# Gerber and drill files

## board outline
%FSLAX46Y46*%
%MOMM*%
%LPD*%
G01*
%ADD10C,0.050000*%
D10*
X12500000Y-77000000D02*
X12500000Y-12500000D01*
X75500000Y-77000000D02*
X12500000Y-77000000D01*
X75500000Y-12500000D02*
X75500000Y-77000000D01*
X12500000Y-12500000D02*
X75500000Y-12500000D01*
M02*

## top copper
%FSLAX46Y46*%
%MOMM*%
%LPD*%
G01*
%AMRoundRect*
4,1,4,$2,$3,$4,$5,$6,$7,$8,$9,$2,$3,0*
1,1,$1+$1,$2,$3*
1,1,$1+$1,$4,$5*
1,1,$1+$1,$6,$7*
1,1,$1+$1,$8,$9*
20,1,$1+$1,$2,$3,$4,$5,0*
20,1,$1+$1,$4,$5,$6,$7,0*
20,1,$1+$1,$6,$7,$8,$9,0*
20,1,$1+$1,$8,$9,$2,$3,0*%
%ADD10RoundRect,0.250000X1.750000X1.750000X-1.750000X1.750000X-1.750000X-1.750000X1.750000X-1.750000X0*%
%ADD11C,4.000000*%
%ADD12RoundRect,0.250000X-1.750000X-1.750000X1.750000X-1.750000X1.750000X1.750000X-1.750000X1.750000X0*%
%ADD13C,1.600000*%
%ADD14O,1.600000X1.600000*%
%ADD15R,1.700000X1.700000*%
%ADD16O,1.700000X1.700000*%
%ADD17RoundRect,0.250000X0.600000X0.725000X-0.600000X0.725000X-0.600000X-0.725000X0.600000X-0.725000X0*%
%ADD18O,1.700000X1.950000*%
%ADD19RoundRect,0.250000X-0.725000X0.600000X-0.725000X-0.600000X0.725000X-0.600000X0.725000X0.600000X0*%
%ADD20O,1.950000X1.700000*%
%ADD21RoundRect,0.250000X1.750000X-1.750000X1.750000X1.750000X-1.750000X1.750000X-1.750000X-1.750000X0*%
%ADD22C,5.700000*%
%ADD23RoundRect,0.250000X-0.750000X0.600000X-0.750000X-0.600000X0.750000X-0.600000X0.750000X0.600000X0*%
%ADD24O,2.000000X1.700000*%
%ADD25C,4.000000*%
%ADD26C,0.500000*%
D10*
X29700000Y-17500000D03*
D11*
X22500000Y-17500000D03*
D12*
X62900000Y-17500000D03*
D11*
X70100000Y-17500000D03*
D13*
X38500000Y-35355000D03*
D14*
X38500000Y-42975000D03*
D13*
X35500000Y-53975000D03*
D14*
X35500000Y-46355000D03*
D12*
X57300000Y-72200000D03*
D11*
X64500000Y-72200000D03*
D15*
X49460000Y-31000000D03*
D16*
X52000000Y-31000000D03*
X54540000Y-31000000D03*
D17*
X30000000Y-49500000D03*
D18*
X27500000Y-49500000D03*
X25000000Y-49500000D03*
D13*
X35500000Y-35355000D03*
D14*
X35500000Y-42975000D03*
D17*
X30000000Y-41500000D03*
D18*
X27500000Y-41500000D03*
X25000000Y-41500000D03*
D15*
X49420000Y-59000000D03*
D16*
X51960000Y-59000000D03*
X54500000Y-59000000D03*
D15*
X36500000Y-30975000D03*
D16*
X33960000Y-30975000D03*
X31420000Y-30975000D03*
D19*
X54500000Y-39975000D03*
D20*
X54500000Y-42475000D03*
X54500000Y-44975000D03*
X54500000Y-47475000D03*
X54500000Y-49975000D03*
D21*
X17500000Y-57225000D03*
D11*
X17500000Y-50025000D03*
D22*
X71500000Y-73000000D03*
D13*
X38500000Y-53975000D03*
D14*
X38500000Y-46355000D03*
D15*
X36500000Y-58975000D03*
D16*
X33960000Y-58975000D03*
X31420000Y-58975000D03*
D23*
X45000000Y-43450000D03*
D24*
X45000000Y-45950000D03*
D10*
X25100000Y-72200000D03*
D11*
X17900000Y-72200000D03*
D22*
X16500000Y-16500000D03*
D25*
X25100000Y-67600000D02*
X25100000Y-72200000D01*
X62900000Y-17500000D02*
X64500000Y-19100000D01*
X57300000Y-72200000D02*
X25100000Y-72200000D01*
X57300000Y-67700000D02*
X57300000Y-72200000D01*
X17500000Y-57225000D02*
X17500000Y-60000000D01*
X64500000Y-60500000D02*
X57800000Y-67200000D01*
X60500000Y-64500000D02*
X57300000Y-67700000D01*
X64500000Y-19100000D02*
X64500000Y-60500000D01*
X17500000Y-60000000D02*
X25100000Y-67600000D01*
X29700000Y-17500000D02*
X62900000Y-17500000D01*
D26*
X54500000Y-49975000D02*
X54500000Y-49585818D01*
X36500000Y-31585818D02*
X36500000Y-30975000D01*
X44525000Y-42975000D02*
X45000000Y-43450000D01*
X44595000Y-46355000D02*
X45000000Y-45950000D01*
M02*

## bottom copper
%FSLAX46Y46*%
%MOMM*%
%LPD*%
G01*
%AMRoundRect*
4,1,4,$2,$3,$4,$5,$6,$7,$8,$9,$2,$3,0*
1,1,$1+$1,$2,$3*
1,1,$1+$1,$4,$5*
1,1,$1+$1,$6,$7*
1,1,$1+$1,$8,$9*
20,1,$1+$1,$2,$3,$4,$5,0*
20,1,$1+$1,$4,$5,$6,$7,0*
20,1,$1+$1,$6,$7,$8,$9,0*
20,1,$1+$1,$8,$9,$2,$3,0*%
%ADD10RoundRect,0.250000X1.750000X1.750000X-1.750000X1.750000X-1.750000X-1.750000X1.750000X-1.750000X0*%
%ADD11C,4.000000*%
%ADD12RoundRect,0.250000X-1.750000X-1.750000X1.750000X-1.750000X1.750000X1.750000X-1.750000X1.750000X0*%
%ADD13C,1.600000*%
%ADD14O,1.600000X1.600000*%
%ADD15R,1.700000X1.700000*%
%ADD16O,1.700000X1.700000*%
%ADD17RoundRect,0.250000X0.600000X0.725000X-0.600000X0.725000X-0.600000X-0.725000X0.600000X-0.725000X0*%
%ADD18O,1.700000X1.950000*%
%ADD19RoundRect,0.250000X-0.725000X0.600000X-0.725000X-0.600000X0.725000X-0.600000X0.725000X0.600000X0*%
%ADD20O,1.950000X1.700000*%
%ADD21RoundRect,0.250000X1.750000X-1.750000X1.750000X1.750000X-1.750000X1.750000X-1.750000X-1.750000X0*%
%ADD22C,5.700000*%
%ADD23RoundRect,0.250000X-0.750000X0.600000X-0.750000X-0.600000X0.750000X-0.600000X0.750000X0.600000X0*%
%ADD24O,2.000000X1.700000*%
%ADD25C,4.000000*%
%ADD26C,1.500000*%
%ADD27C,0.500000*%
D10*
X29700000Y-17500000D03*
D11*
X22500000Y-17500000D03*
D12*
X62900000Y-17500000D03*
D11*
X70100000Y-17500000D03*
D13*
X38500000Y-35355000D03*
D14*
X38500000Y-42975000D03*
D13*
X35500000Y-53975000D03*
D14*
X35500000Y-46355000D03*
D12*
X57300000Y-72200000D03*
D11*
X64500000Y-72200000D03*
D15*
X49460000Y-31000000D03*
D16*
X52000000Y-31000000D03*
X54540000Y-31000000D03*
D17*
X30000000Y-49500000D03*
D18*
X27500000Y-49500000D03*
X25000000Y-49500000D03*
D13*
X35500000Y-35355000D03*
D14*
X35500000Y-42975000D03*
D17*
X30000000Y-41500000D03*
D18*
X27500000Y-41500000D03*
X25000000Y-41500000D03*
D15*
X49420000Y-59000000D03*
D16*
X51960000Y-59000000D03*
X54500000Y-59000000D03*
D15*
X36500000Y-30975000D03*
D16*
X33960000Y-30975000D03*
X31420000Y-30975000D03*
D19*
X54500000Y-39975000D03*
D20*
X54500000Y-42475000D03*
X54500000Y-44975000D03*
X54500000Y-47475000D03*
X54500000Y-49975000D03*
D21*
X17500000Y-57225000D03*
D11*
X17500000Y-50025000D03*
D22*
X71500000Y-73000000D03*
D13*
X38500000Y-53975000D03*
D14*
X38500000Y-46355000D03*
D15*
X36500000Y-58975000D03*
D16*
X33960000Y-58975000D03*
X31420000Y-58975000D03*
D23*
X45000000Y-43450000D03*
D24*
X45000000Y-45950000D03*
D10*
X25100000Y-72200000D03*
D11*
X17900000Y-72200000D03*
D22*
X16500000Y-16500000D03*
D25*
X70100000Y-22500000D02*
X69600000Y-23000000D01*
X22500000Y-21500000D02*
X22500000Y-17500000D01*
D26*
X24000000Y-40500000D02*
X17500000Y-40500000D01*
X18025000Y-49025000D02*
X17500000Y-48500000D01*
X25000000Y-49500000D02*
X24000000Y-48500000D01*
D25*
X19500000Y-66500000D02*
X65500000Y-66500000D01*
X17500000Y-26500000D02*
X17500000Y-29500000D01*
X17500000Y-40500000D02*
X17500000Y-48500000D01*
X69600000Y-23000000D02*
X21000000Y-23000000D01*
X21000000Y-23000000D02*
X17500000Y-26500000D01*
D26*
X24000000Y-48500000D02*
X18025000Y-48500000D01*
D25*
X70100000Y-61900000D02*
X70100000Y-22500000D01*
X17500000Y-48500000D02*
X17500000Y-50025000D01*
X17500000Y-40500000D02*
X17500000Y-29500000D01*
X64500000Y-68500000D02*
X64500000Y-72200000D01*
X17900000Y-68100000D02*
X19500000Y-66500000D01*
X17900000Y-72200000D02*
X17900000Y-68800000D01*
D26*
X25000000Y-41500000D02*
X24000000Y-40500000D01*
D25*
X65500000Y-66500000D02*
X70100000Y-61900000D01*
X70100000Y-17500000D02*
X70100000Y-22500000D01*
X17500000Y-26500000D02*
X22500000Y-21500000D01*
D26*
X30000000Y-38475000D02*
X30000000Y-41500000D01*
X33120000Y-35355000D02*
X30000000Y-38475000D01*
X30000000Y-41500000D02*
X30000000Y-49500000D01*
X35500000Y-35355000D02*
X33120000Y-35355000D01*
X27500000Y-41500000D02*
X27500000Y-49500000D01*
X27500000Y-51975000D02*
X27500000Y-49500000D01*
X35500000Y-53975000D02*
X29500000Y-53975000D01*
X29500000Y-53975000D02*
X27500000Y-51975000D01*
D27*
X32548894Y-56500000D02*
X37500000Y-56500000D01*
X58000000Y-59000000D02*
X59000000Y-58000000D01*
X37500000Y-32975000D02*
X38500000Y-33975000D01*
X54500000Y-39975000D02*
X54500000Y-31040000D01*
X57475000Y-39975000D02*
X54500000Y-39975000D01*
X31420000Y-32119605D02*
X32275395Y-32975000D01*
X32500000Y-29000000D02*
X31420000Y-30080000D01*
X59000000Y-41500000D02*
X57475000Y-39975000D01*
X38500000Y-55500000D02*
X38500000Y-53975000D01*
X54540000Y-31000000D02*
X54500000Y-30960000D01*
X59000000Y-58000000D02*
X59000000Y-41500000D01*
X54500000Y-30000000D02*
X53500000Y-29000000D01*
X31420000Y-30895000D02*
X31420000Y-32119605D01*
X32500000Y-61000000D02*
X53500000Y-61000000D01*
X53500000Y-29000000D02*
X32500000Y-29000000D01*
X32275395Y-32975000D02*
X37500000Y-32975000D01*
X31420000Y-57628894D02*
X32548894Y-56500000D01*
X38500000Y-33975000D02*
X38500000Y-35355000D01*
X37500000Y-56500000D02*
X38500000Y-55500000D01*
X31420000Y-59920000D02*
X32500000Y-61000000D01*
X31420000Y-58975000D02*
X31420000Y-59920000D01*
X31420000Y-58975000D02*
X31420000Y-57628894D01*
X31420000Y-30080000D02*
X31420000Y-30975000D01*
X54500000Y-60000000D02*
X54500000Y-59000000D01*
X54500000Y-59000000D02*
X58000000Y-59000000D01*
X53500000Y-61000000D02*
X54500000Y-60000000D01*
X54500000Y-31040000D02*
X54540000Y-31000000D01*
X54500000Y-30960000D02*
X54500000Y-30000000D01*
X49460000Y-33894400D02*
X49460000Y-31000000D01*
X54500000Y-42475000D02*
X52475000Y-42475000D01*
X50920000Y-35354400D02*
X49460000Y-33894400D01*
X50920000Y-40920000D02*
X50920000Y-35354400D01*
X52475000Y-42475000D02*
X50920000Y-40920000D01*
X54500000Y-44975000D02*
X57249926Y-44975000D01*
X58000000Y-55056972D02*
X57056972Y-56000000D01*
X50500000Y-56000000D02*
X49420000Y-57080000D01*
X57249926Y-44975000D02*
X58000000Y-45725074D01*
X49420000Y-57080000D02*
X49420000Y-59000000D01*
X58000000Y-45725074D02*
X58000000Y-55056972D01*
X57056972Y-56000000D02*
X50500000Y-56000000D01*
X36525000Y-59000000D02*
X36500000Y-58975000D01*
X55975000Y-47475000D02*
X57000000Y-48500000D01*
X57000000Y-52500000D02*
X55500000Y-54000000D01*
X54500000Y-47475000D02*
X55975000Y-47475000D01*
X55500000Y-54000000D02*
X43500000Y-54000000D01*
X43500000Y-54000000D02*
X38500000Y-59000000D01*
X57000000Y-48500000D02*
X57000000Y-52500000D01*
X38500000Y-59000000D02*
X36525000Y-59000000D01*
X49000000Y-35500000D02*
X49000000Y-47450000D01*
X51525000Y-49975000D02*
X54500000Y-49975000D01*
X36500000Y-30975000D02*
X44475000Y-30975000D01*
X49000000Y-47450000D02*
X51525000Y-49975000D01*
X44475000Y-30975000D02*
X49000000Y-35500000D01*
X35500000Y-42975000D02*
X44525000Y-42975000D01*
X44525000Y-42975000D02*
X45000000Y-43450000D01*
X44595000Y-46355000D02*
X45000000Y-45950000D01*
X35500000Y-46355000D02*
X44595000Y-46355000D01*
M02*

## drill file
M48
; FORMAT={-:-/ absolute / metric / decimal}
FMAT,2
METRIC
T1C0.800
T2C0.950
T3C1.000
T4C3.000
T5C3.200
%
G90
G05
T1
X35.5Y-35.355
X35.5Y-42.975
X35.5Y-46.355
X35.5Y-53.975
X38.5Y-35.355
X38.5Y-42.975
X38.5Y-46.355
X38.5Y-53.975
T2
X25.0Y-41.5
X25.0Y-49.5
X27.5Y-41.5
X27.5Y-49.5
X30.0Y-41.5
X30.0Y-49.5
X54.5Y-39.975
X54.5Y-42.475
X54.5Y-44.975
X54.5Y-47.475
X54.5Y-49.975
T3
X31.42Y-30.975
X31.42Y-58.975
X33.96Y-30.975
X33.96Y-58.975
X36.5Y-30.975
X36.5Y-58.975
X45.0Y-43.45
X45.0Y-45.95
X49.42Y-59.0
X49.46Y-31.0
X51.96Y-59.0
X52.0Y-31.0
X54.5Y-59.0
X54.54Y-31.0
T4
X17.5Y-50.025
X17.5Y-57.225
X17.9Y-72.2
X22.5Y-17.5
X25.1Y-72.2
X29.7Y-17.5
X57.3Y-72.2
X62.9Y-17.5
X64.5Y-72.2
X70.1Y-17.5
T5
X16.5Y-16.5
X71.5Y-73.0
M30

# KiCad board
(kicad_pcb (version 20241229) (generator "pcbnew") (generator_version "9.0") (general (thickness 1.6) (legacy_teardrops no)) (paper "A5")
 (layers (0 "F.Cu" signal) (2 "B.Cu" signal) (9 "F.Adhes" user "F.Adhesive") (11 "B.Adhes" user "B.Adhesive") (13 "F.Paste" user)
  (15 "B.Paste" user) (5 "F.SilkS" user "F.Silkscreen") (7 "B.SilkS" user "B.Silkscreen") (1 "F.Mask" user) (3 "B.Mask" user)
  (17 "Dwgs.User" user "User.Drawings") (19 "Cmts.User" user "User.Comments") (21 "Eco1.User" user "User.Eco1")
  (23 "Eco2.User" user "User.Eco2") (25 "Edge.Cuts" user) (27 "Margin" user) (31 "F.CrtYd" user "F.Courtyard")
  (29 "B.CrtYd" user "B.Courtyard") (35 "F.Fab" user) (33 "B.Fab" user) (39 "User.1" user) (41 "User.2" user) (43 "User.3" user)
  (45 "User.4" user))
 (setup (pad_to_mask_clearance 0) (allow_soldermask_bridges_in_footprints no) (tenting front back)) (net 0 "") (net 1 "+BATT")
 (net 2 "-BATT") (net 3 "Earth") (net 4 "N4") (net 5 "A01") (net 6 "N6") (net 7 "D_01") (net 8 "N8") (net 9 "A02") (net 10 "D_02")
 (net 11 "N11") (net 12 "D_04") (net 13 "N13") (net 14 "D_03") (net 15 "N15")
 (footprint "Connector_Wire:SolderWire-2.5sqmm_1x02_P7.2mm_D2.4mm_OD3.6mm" (layer "F.Cu") (at 29.7 17.5 180)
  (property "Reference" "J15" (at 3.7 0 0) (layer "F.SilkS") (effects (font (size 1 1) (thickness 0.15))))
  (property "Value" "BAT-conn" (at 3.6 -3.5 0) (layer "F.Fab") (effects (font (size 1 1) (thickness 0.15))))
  (pad "1" thru_hole roundrect (at 0 0 180) (size 4 4) (drill 3) (layers "*.Cu" "*.Mask") (remove_unused_layers no)
   (roundrect_rratio 0.0625) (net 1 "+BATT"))
  (pad "2" thru_hole circle (at 7.2 0 180) (size 4 4) (drill 3) (layers "*.Cu" "*.Mask") (remove_unused_layers no) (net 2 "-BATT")))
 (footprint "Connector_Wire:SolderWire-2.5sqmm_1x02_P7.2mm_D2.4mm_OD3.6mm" (layer "F.Cu") (at 62.9 17.5)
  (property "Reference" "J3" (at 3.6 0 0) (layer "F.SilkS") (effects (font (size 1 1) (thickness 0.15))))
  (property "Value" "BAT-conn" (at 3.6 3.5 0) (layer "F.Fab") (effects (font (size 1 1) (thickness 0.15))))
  (pad "1" thru_hole roundrect (at 0 0) (size 4 4) (drill 3) (layers "*.Cu" "*.Mask") (remove_unused_layers no) (roundrect_rratio 0.0625)
   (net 1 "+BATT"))
  (pad "2" thru_hole circle (at 7.2 0) (size 4 4) (drill 3) (layers "*.Cu" "*.Mask") (remove_unused_layers no) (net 2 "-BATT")))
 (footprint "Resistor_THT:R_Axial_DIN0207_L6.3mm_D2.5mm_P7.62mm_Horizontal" (layer "F.Cu") (at 38.5 35.355 -90)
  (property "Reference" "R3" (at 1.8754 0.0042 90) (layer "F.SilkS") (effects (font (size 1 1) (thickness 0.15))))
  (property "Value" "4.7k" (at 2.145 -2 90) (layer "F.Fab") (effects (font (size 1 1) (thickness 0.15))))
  (pad "1" thru_hole circle (at 0 0 270) (size 1.6 1.6) (drill 0.8) (layers "*.Cu" "*.Mask") (remove_unused_layers no) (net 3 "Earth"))
  (pad "2" thru_hole oval (at 7.62 0 270) (size 1.6 1.6) (drill 0.8) (layers "*.Cu" "*.Mask") (remove_unused_layers no) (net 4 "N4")))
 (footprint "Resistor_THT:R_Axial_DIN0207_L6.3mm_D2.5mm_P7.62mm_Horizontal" (layer "F.Cu") (at 35.5 53.975 90)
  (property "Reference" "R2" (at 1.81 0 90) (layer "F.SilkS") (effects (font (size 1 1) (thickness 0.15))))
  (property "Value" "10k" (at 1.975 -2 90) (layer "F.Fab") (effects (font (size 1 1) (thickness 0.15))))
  (pad "1" thru_hole circle (at 0 0 90) (size 1.6 1.6) (drill 0.8) (layers "*.Cu" "*.Mask") (remove_unused_layers no) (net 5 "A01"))
  (pad "2" thru_hole oval (at 7.62 0 90) (size 1.6 1.6) (drill 0.8) (layers "*.Cu" "*.Mask") (remove_unused_layers no) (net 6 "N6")))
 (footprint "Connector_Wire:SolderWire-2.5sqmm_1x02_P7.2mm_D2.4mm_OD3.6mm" (layer "F.Cu") (at 57.3 72.2)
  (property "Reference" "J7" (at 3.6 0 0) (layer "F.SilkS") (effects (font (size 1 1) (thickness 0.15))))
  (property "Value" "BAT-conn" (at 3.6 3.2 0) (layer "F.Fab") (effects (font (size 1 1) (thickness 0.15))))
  (pad "1" thru_hole roundrect (at 0 0) (size 4 4) (drill 3) (layers "*.Cu" "*.Mask") (remove_unused_layers no) (roundrect_rratio 0.0625)
   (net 1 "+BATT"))
  (pad "2" thru_hole circle (at 7.2 0) (size 4 4) (drill 3) (layers "*.Cu" "*.Mask") (remove_unused_layers no) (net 2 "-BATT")))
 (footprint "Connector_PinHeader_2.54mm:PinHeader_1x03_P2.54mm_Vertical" (layer "F.Cu") (at 49.46 31 90)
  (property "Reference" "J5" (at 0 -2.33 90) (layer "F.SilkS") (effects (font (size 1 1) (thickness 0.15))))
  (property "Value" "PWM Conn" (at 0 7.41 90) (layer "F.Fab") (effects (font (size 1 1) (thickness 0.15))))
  (pad "1" thru_hole rect (at 0 0 90) (size 1.7 1.7) (drill 1) (layers "*.Cu" "*.Mask") (remove_unused_layers no) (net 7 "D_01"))
  (pad "2" thru_hole oval (at 0 2.54 90) (size 1.7 1.7) (drill 1) (layers "*.Cu" "*.Mask") (remove_unused_layers no) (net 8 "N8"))
  (pad "3" thru_hole oval (at 0 5.08 90) (size 1.7 1.7) (drill 1) (layers "*.Cu" "*.Mask") (remove_unused_layers no) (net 3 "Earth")))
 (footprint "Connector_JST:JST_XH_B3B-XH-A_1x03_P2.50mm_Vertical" (layer "F.Cu") (at 30 49.5 180)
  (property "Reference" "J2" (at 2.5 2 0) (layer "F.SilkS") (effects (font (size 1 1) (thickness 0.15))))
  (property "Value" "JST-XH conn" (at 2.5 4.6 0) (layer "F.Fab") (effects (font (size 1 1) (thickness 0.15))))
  (pad "1" thru_hole roundrect (at 0 0 180) (size 1.7 1.95) (drill 0.95) (layers "*.Cu" "*.Mask") (remove_unused_layers no)
   (roundrect_rratio 0.147059) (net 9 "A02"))
  (pad "2" thru_hole oval (at 2.5 0 180) (size 1.7 1.95) (drill 0.95) (layers "*.Cu" "*.Mask") (remove_unused_layers no) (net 5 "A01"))
  (pad "3" thru_hole oval (at 5 0 180) (size 1.7 1.95) (drill 0.95) (layers "*.Cu" "*.Mask") (remove_unused_layers no) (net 2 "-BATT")))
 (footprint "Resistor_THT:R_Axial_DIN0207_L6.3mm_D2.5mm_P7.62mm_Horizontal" (layer "F.Cu") (at 35.5 35.355 -90)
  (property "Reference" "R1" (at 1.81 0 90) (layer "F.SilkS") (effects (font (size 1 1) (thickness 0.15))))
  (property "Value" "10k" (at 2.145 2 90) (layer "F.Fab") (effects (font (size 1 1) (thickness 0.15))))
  (pad "1" thru_hole circle (at 0 0 270) (size 1.6 1.6) (drill 0.8) (layers "*.Cu" "*.Mask") (remove_unused_layers no) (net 9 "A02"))
  (pad "2" thru_hole oval (at 7.62 0 270) (size 1.6 1.6) (drill 0.8) (layers "*.Cu" "*.Mask") (remove_unused_layers no) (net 4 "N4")))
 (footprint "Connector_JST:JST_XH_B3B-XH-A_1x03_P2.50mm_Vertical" (layer "F.Cu") (at 30 41.5 180)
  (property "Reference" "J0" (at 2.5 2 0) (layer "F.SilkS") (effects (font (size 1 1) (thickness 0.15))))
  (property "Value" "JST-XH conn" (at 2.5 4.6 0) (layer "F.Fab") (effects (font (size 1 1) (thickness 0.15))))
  (pad "1" thru_hole roundrect (at 0 0 180) (size 1.7 1.95) (drill 0.95) (layers "*.Cu" "*.Mask") (remove_unused_layers no)
   (roundrect_rratio 0.147059) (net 9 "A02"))
  (pad "2" thru_hole oval (at 2.5 0 180) (size 1.7 1.95) (drill 0.95) (layers "*.Cu" "*.Mask") (remove_unused_layers no) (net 5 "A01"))
  (pad "3" thru_hole oval (at 5 0 180) (size 1.7 1.95) (drill 0.95) (layers "*.Cu" "*.Mask") (remove_unused_layers no) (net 2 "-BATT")))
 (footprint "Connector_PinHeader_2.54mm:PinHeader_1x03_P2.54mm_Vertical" (layer "F.Cu") (at 49.42 59 90)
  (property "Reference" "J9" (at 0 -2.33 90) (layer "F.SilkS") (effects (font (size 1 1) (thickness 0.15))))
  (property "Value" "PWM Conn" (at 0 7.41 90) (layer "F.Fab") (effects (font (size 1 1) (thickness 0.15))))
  (pad "1" thru_hole rect (at 0 0 90) (size 1.7 1.7) (drill 1) (layers "*.Cu" "*.Mask") (remove_unused_layers no) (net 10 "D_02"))
  (pad "2" thru_hole oval (at 0 2.54 90) (size 1.7 1.7) (drill 1) (layers "*.Cu" "*.Mask") (remove_unused_layers no) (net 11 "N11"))
  (pad "3" thru_hole oval (at 0 5.08 90) (size 1.7 1.7) (drill 1) (layers "*.Cu" "*.Mask") (remove_unused_layers no) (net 3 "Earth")))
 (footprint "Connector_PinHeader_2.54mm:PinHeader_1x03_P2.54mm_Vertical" (layer "F.Cu") (at 36.5 30.975 -90)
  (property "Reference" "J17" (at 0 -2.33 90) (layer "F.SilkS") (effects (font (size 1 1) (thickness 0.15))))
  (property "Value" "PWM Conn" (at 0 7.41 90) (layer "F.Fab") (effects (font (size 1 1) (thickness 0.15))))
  (pad "1" thru_hole rect (at 0 0 270) (size 1.7 1.7) (drill 1) (layers "*.Cu" "*.Mask") (remove_unused_layers no) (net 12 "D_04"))
  (pad "2" thru_hole oval (at 0 2.54 270) (size 1.7 1.7) (drill 1) (layers "*.Cu" "*.Mask") (remove_unused_layers no) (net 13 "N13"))
  (pad "3" thru_hole oval (at 0 5.08 270) (size 1.7 1.7) (drill 1) (layers "*.Cu" "*.Mask") (remove_unused_layers no) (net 3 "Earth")))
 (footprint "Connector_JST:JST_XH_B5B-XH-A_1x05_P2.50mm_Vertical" (layer "F.Cu") (at 54.5 39.975 -90)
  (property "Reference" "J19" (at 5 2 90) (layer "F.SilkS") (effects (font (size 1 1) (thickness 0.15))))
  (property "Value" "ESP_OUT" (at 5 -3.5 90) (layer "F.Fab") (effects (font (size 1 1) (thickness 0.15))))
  (pad "1" thru_hole roundrect (at 0 0 270) (size 1.7 1.95) (drill 0.95) (layers "*.Cu" "*.Mask") (remove_unused_layers no)
   (roundrect_rratio 0.147059) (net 3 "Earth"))
  (pad "2" thru_hole oval (at 2.5 0 270) (size 1.7 1.95) (drill 0.95) (layers "*.Cu" "*.Mask") (remove_unused_layers no) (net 7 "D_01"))
  (pad "3" thru_hole oval (at 5 0 270) (size 1.7 1.95) (drill 0.95) (layers "*.Cu" "*.Mask") (remove_unused_layers no) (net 10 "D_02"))
  (pad "4" thru_hole oval (at 7.5 0 270) (size 1.7 1.95) (drill 0.95) (layers "*.Cu" "*.Mask") (remove_unused_layers no) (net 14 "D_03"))
  (pad "5" thru_hole oval (at 10 0 270) (size 1.7 1.95) (drill 0.95) (layers "*.Cu" "*.Mask") (remove_unused_layers no) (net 12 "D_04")))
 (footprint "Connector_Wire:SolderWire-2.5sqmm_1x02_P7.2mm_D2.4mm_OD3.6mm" (layer "F.Cu") (at 17.5 57.225 90)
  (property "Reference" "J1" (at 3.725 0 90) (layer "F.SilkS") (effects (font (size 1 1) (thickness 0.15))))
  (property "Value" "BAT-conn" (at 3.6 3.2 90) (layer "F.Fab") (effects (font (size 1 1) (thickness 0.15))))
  (pad "1" thru_hole roundrect (at 0 0 90) (size 4 4) (drill 3) (layers "*.Cu" "*.Mask") (remove_unused_layers no) (roundrect_rratio 0.0625)
   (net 1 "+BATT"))
  (pad "2" thru_hole circle (at 7.2 0 90) (size 4 4) (drill 3) (layers "*.Cu" "*.Mask") (remove_unused_layers no) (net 2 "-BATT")))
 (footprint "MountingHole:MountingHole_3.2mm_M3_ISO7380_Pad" (layer "F.Cu") (at 71.5 73)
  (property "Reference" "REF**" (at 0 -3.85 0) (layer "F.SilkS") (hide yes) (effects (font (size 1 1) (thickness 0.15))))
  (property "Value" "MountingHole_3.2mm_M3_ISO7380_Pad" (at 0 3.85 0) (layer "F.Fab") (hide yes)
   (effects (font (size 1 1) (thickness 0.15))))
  (pad "1" thru_hole circle (at 0 0) (size 5.7 5.7) (drill 3.2) (layers "*.Cu" "*.Mask") (remove_unused_layers no)))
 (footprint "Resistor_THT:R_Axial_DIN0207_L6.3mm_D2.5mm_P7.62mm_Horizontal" (layer "F.Cu") (at 38.5 53.975 90)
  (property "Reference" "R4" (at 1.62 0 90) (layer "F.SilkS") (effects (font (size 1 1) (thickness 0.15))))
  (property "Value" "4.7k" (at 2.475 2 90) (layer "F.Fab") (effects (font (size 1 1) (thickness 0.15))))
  (pad "1" thru_hole circle (at 0 0 90) (size 1.6 1.6) (drill 0.8) (layers "*.Cu" "*.Mask") (remove_unused_layers no) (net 3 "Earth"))
  (pad "2" thru_hole oval (at 7.62 0 90) (size 1.6 1.6) (drill 0.8) (layers "*.Cu" "*.Mask") (remove_unused_layers no) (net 6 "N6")))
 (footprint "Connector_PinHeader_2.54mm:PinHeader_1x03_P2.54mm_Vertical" (layer "F.Cu") (at 36.5 58.975 -90)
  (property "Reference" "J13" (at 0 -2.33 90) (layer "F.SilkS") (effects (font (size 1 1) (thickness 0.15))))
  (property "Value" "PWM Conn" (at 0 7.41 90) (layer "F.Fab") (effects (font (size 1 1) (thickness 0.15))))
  (pad "1" thru_hole rect (at 0 0 270) (size 1.7 1.7) (drill 1) (layers "*.Cu" "*.Mask") (remove_unused_layers no) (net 14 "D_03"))
  (pad "2" thru_hole oval (at 0 2.54 270) (size 1.7 1.7) (drill 1) (layers "*.Cu" "*.Mask") (remove_unused_layers no) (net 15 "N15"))
  (pad "3" thru_hole oval (at 0 5.08 270) (size 1.7 1.7) (drill 1) (layers "*.Cu" "*.Mask") (remove_unused_layers no) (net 3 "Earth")))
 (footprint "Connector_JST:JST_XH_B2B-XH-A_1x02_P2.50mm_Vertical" (layer "F.Cu") (at 45 43.45 -90)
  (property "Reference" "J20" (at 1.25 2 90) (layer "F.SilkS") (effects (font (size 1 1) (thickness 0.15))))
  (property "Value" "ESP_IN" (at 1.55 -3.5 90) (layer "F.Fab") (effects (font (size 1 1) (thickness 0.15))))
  (pad "1" thru_hole roundrect (at 0 0 270) (size 1.7 2) (drill 1) (layers "*.Cu" "*.Mask") (remove_unused_layers no)
   (roundrect_rratio 0.147059) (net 4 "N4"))
  (pad "2" thru_hole oval (at 2.5 0 270) (size 1.7 2) (drill 1) (layers "*.Cu" "*.Mask") (remove_unused_layers no) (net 6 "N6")))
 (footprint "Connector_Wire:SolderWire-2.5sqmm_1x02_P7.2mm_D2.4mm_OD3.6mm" (layer "F.Cu") (at 25.1 72.2 180)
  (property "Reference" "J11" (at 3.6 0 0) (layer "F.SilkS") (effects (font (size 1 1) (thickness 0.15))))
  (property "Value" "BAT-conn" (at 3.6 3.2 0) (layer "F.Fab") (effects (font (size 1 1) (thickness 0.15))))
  (pad "1" thru_hole roundrect (at 0 0 180) (size 4 4) (drill 3) (layers "*.Cu" "*.Mask") (remove_unused_layers no)
   (roundrect_rratio 0.0625) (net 1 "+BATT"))
  (pad "2" thru_hole circle (at 7.2 0 180) (size 4 4) (drill 3) (layers "*.Cu" "*.Mask") (remove_unused_layers no) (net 2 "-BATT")))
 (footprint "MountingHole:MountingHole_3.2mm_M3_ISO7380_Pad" (layer "F.Cu") (at 16.5 16.5)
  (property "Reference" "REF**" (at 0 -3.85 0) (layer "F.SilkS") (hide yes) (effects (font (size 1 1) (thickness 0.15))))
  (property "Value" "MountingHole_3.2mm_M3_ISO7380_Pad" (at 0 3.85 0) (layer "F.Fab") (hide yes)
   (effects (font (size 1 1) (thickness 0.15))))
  (pad "1" thru_hole circle (at 0 0) (size 5.7 5.7) (drill 3.2) (layers "*.Cu" "*.Mask") (remove_unused_layers no)))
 (gr_line (start 12.5 77) (end 12.5 12.5) (stroke (width 0.05) (type default)) (layer "Edge.Cuts"))
 (gr_line (start 75.5 77) (end 12.5 77) (stroke (width 0.05) (type default)) (layer "Edge.Cuts"))
 (gr_line (start 75.5 12.5) (end 75.5 77) (stroke (width 0.05) (type default)) (layer "Edge.Cuts"))
 (gr_line (start 12.5 12.5) (end 75.5 12.5) (stroke (width 0.05) (type default)) (layer "Edge.Cuts"))
 (segment (start 70.1 22.5) (end 69.6 23) (width 4) (layer "B.Cu") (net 2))
 (segment (start 22.5 21.5) (end 22.5 17.5) (width 4) (layer "B.Cu") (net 2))
 (segment (start 24 40.5) (end 17.5 40.5) (width 1.5) (layer "B.Cu") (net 2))
 (segment (start 18.025 49.025) (end 17.5 48.5) (width 1.5) (layer "B.Cu") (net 2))
 (segment (start 25 49.5) (end 24 48.5) (width 1.5) (layer "B.Cu") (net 2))
 (segment (start 19.5 66.5) (end 65.5 66.5) (width 4) (layer "B.Cu") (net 2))
 (segment (start 17.5 26.5) (end 17.5 29.5) (width 4) (layer "B.Cu") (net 2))
 (segment (start 17.5 40.5) (end 17.5 48.5) (width 4) (layer "B.Cu") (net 2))
 (segment (start 69.6 23) (end 21 23) (width 4) (layer "B.Cu") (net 2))
 (segment (start 21 23) (end 17.5 26.5) (width 4) (layer "B.Cu") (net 2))
 (segment (start 24 48.5) (end 18.025 48.5) (width 1.5) (layer "B.Cu") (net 2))
 (segment (start 70.1 61.9) (end 70.1 22.5) (width 4) (layer "B.Cu") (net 2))
 (segment (start 17.5 48.5) (end 17.5 50.025) (width 4) (layer "B.Cu") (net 2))
 (segment (start 17.5 40.5) (end 17.5 29.5) (width 4) (layer "B.Cu") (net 2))
 (segment (start 64.5 68.5) (end 64.5 72.2) (width 4) (layer "B.Cu") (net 2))
 (segment (start 17.9 68.1) (end 19.5 66.5) (width 4) (layer "B.Cu") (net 2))
 (segment (start 17.9 72.2) (end 17.9 68.8) (width 4) (layer "B.Cu") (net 2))
 (segment (start 25 41.5) (end 24 40.5) (width 1.5) (layer "B.Cu") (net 2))
 (segment (start 65.5 66.5) (end 70.1 61.9) (width 4) (layer "B.Cu") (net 2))
 (segment (start 70.1 17.5) (end 70.1 22.5) (width 4) (layer "B.Cu") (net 2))
 (segment (start 17.5 26.5) (end 22.5 21.5) (width 4) (layer "B.Cu") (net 2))
 (segment (start 30 38.475) (end 30 41.5) (width 1.5) (layer "B.Cu") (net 9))
 (segment (start 33.12 35.355) (end 30 38.475) (width 1.5) (layer "B.Cu") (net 9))
 (segment (start 30 41.5) (end 30 49.5) (width 1.5) (layer "B.Cu") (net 9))
 (segment (start 35.5 35.355) (end 33.12 35.355) (width 1.5) (layer "B.Cu") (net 9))
 (segment (start 27.5 41.5) (end 27.5 49.5) (width 1.5) (layer "B.Cu") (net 5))
 (segment (start 27.5 51.975) (end 27.5 49.5) (width 1.5) (layer "B.Cu") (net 5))
 (segment (start 35.5 53.975) (end 29.5 53.975) (width 1.5) (layer "B.Cu") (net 5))
 (segment (start 29.5 53.975) (end 27.5 51.975) (width 1.5) (layer "B.Cu") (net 5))
 (segment (start 25.1 67.6) (end 25.1 72.2) (width 4) (layer "F.Cu") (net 1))
 (segment (start 62.9 17.5) (end 64.5 19.1) (width 4) (layer "F.Cu") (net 1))
 (segment (start 57.3 72.2) (end 25.1 72.2) (width 4) (layer "F.Cu") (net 1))
 (segment (start 57.3 67.7) (end 57.3 72.2) (width 4) (layer "F.Cu") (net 1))
 (segment (start 17.5 57.225) (end 17.5 60) (width 4) (layer "F.Cu") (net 1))
 (segment (start 64.5 60.5) (end 57.8 67.2) (width 4) (layer "F.Cu") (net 1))
 (segment (start 60.5 64.5) (end 57.3 67.7) (width 4) (layer "F.Cu") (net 1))
 (segment (start 64.5 19.1) (end 64.5 60.5) (width 4) (layer "F.Cu") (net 1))
 (segment (start 17.5 60) (end 25.1 67.6) (width 4) (layer "F.Cu") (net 1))
 (segment (start 29.7 17.5) (end 62.9 17.5) (width 4) (layer "F.Cu") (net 1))
 (segment (start 32.548894 56.5) (end 37.5 56.5) (width 0.5) (layer "B.Cu") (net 3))
 (segment (start 58 59) (end 59 58) (width 0.5) (layer "B.Cu") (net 3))
 (segment (start 37.5 32.975) (end 38.5 33.975) (width 0.5) (layer "B.Cu") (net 3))
 (segment (start 54.5 39.975) (end 54.5 31.04) (width 0.5) (layer "B.Cu") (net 3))
 (segment (start 57.475 39.975) (end 54.5 39.975) (width 0.5) (layer "B.Cu") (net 3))
 (segment (start 31.42 32.119605) (end 32.275395 32.975) (width 0.5) (layer "B.Cu") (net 3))
 (segment (start 32.5 29) (end 31.42 30.08) (width 0.5) (layer "B.Cu") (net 3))
 (segment (start 59 41.5) (end 57.475 39.975) (width 0.5) (layer "B.Cu") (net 3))
 (segment (start 38.5 55.5) (end 38.5 53.975) (width 0.5) (layer "B.Cu") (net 3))
 (segment (start 54.54 31) (end 54.5 30.96) (width 0.5) (layer "B.Cu") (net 3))
 (segment (start 59 58) (end 59 41.5) (width 0.5) (layer "B.Cu") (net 3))
 (segment (start 54.5 30) (end 53.5 29) (width 0.5) (layer "B.Cu") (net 3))
 (segment (start 31.42 30.895) (end 31.42 32.119605) (width 0.5) (layer "B.Cu") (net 3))
 (segment (start 32.5 61) (end 53.5 61) (width 0.5) (layer "B.Cu") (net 3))
 (segment (start 53.5 29) (end 32.5 29) (width 0.5) (layer "B.Cu") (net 3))
 (segment (start 32.275395 32.975) (end 37.5 32.975) (width 0.5) (layer "B.Cu") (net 3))
 (segment (start 31.42 57.628894) (end 32.548894 56.5) (width 0.5) (layer "B.Cu") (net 3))
 (segment (start 38.5 33.975) (end 38.5 35.355) (width 0.5) (layer "B.Cu") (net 3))
 (segment (start 37.5 56.5) (end 38.5 55.5) (width 0.5) (layer "B.Cu") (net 3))
 (segment (start 31.42 59.92) (end 32.5 61) (width 0.5) (layer "B.Cu") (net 3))
 (segment (start 31.42 58.975) (end 31.42 59.92) (width 0.5) (layer "B.Cu") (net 3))
 (segment (start 31.42 58.975) (end 31.42 57.628894) (width 0.5) (layer "B.Cu") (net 3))
 (segment (start 31.42 30.08) (end 31.42 30.975) (width 0.5) (layer "B.Cu") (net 3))
 (segment (start 54.5 60) (end 54.5 59) (width 0.5) (layer "B.Cu") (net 3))
 (segment (start 54.5 59) (end 58 59) (width 0.5) (layer "B.Cu") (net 3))
 (segment (start 53.5 61) (end 54.5 60) (width 0.5) (layer "B.Cu") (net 3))
 (segment (start 54.5 31.04) (end 54.54 31) (width 0.5) (layer "B.Cu") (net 3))
 (segment (start 54.5 30.96) (end 54.5 30) (width 0.5) (layer "B.Cu") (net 3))
 (segment (start 49.46 33.8944) (end 49.46 31) (width 0.5) (layer "B.Cu") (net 7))
 (segment (start 54.5 42.475) (end 52.475 42.475) (width 0.5) (layer "B.Cu") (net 7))
 (segment (start 50.92 35.3544) (end 49.46 33.8944) (width 0.5) (layer "B.Cu") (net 7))
 (segment (start 50.92 40.92) (end 50.92 35.3544) (width 0.5) (layer "B.Cu") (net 7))
 (segment (start 52.475 42.475) (end 50.92 40.92) (width 0.5) (layer "B.Cu") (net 7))
 (segment (start 54.5 44.975) (end 57.249926 44.975) (width 0.5) (layer "B.Cu") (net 10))
 (segment (start 58 55.056972) (end 57.056972 56) (width 0.5) (layer "B.Cu") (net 10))
 (segment (start 50.5 56) (end 49.42 57.08) (width 0.5) (layer "B.Cu") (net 10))
 (segment (start 57.249926 44.975) (end 58 45.725074) (width 0.5) (layer "B.Cu") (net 10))
 (segment (start 49.42 57.08) (end 49.42 59) (width 0.5) (layer "B.Cu") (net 10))
 (segment (start 58 45.725074) (end 58 55.056972) (width 0.5) (layer "B.Cu") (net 10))
 (segment (start 57.056972 56) (end 50.5 56) (width 0.5) (layer "B.Cu") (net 10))
 (segment (start 36.525 59) (end 36.5 58.975) (width 0.5) (layer "B.Cu") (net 14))
 (segment (start 55.975 47.475) (end 57 48.5) (width 0.5) (layer "B.Cu") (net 14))
 (segment (start 57 52.5) (end 55.5 54) (width 0.5) (layer "B.Cu") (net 14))
 (segment (start 54.5 47.475) (end 55.975 47.475) (width 0.5) (layer "B.Cu") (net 14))
 (segment (start 55.5 54) (end 43.5 54) (width 0.5) (layer "B.Cu") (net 14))
 (segment (start 43.5 54) (end 38.5 59) (width 0.5) (layer "B.Cu") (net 14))
 (segment (start 57 48.5) (end 57 52.5) (width 0.5) (layer "B.Cu") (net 14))
 (segment (start 38.5 59) (end 36.525 59) (width 0.5) (layer "B.Cu") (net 14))
 (segment (start 54.5 49.975) (end 54.5 49.585818) (width 0.5) (layer "F.Cu") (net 12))
 (segment (start 36.5 31.585818) (end 36.5 30.975) (width 0.5) (layer "F.Cu") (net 12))
 (segment (start 49 35.5) (end 49 47.45) (width 0.5) (layer "B.Cu") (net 12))
 (segment (start 51.525 49.975) (end 54.5 49.975) (width 0.5) (layer "B.Cu") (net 12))
 (segment (start 36.5 30.975) (end 44.475 30.975) (width 0.5) (layer "B.Cu") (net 12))
 (segment (start 49 47.45) (end 51.525 49.975) (width 0.5) (layer "B.Cu") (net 12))
 (segment (start 44.475 30.975) (end 49 35.5) (width 0.5) (layer "B.Cu") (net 12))
 (segment (start 44.525 42.975) (end 45 43.45) (width 0.5) (layer "F.Cu") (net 4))
 (segment (start 35.5 42.975) (end 44.525 42.975) (width 0.5) (layer "B.Cu") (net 4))
 (segment (start 44.525 42.975) (end 45 43.45) (width 0.5) (layer "B.Cu") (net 4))
 (segment (start 44.595 46.355) (end 45 45.95) (width 0.5) (layer "F.Cu") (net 6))
 (segment (start 44.595 46.355) (end 45 45.95) (width 0.5) (layer "B.Cu") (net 6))
 (segment (start 35.5 46.355) (end 44.595 46.355) (width 0.5) (layer "B.Cu") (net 6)))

